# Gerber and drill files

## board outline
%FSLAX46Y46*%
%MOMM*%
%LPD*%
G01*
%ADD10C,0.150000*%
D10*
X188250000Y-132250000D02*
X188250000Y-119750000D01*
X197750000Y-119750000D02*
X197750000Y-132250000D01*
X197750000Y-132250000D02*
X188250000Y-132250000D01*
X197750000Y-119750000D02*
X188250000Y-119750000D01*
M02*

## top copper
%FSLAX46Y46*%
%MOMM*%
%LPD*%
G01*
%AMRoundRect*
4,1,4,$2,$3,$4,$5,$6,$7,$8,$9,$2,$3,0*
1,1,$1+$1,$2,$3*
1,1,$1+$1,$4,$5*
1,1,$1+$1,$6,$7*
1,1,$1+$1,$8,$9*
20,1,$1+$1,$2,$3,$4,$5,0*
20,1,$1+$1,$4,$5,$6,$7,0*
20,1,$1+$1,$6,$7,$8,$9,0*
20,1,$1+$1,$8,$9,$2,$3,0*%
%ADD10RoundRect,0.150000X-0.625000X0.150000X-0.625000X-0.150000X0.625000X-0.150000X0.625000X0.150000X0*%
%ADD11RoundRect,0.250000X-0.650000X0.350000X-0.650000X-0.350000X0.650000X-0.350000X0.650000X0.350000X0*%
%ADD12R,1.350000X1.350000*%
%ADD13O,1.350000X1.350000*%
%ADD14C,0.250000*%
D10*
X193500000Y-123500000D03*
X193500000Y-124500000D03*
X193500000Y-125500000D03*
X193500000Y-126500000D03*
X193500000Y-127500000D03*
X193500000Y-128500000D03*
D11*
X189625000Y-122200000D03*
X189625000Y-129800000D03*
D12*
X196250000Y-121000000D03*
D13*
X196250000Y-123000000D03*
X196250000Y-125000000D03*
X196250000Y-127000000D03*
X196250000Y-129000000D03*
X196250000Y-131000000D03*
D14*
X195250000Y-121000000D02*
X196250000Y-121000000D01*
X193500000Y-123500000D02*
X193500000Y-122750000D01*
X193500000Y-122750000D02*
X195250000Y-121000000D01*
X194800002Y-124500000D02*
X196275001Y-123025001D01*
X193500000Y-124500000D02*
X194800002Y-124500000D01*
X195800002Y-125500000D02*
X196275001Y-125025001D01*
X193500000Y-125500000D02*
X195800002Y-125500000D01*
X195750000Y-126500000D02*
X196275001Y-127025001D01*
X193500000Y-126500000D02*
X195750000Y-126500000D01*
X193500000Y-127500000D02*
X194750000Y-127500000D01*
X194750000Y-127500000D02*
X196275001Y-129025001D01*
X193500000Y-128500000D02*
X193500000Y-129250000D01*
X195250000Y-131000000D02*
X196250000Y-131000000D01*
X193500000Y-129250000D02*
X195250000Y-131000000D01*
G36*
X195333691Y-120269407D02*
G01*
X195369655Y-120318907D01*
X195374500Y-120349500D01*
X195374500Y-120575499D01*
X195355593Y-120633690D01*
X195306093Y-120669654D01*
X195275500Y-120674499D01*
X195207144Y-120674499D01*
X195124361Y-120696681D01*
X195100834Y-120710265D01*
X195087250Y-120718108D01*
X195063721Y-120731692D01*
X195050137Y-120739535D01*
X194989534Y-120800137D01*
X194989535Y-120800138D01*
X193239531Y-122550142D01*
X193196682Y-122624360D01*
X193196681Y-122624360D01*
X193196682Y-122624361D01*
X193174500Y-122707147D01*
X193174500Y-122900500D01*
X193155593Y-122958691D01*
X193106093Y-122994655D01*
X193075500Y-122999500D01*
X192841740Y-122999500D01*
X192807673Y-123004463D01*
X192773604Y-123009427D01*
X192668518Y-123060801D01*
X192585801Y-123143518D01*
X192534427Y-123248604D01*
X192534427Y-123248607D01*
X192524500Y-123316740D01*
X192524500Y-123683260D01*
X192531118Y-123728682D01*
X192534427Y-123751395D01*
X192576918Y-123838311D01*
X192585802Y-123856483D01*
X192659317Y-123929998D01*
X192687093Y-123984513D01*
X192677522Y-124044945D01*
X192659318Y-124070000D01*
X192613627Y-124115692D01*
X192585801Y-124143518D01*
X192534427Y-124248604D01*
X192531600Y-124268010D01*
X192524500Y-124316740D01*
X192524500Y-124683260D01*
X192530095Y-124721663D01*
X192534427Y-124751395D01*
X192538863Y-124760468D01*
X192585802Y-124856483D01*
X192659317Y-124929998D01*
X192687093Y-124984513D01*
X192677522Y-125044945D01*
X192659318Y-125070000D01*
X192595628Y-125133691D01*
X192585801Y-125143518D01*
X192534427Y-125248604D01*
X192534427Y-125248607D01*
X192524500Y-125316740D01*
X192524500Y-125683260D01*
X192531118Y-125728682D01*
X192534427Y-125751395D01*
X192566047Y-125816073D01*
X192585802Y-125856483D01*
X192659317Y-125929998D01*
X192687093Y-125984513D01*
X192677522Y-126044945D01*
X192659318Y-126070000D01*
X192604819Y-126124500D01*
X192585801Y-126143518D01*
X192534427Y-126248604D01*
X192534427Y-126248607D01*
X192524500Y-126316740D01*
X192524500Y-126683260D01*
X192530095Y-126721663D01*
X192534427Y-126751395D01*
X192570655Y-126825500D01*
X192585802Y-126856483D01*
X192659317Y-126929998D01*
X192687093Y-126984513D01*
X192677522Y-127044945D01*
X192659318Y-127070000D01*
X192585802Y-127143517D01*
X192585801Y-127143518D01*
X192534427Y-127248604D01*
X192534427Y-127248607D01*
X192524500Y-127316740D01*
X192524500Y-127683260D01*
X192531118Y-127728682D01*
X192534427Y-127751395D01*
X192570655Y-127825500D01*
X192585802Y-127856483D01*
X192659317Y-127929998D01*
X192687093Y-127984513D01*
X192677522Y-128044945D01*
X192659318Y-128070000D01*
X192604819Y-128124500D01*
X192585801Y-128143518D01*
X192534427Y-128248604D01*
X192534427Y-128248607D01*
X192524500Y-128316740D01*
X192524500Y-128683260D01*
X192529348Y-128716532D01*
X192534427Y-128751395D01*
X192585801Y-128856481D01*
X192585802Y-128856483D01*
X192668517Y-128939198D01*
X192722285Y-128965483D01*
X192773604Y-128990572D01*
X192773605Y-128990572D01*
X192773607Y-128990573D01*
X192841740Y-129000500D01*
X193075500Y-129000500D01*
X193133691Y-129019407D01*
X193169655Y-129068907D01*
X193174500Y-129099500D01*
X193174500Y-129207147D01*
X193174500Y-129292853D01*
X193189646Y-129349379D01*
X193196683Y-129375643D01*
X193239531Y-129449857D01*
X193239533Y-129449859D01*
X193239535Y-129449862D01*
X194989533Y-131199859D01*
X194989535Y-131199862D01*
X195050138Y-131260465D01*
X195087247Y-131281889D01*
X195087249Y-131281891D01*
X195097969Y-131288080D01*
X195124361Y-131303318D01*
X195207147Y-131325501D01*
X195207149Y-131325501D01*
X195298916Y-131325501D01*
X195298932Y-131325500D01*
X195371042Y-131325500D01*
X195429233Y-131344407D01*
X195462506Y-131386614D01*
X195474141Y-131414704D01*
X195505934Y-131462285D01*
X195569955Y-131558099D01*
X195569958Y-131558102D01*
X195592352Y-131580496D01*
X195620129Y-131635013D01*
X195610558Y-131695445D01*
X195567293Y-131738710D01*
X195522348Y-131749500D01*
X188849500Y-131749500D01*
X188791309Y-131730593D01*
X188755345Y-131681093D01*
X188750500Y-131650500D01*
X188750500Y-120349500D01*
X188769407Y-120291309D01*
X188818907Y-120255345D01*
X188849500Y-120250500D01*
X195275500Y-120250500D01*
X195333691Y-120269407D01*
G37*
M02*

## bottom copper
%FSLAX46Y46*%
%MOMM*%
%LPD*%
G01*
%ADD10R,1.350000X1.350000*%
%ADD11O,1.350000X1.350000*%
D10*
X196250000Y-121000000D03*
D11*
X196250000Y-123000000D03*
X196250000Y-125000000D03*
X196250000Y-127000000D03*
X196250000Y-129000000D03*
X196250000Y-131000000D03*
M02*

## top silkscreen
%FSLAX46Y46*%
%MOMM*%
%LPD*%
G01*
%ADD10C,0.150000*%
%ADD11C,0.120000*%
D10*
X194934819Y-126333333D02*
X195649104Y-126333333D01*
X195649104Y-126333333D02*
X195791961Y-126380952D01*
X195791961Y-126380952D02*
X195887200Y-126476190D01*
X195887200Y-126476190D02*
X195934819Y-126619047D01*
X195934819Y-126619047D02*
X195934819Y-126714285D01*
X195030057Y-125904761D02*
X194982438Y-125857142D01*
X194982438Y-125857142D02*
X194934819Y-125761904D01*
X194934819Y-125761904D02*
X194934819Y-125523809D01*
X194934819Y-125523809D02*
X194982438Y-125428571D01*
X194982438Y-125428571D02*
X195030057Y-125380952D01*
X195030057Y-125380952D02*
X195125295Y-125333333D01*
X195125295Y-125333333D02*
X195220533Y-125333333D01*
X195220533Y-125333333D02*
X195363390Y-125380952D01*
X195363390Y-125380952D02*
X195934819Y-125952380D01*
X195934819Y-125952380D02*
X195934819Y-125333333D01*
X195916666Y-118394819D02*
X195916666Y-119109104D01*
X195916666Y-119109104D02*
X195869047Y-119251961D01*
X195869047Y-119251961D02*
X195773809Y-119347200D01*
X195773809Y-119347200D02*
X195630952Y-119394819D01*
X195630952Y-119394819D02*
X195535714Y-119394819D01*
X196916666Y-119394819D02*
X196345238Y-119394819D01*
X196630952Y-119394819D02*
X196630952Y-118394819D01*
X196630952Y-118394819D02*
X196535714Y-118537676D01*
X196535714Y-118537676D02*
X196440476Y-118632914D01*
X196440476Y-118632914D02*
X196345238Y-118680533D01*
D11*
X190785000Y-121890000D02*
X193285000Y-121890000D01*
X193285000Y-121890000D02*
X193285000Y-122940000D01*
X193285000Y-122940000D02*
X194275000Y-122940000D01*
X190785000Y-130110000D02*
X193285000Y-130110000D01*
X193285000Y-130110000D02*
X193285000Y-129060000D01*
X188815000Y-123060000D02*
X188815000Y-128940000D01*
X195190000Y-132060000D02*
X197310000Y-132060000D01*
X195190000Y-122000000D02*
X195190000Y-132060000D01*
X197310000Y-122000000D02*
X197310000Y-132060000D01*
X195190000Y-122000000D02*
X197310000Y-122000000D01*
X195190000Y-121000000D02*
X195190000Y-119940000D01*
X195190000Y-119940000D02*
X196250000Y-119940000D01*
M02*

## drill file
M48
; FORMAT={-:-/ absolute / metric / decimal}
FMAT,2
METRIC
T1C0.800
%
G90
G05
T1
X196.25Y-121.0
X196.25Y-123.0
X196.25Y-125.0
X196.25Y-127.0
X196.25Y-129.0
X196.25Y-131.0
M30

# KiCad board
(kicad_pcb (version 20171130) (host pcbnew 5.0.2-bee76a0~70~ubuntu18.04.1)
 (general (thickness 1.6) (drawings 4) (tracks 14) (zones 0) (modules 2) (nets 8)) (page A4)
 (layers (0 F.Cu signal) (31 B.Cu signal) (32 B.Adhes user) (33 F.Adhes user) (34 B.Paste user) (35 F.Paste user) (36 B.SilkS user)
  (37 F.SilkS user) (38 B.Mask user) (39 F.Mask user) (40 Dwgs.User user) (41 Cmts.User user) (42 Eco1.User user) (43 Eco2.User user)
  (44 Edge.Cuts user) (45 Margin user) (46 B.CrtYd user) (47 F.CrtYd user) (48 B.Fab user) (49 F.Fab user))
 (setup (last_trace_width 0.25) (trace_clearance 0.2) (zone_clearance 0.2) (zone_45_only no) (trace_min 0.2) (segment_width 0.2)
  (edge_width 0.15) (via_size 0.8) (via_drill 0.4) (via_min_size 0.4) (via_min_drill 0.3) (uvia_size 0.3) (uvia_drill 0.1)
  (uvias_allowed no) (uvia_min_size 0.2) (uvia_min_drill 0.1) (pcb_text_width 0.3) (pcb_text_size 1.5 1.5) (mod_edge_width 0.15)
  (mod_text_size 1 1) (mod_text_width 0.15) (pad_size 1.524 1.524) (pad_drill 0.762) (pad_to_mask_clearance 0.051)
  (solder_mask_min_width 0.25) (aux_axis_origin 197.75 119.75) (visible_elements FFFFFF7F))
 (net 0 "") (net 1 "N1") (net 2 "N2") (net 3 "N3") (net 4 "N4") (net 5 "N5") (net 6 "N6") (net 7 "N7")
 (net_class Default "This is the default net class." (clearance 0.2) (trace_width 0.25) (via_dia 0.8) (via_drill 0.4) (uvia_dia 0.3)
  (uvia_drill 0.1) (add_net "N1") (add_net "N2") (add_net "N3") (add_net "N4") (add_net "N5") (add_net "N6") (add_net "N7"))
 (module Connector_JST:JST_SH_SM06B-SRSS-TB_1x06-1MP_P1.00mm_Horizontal (layer F.Cu) (at 191.5 126 270)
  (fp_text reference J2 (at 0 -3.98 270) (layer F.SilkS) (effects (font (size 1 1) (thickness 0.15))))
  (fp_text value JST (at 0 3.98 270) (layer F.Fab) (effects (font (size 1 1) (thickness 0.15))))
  (fp_line (start -4.11 0.715) (end -4.11 -1.785) (layer F.SilkS) (width 0.12))
  (fp_line (start -4.11 -1.785) (end -3.06 -1.785) (layer F.SilkS) (width 0.12))
  (fp_line (start -3.06 -1.785) (end -3.06 -2.775) (layer F.SilkS) (width 0.12))
  (fp_line (start 4.11 0.715) (end 4.11 -1.785) (layer F.SilkS) (width 0.12))
  (fp_line (start 4.11 -1.785) (end 3.06 -1.785) (layer F.SilkS) (width 0.12))
  (fp_line (start -2.94 2.685) (end 2.94 2.685) (layer F.SilkS) (width 0.12))
  (pad 1 smd roundrect (at -2.5 -2 270) (size 0.6 1.55) (layers F.Cu F.Paste F.Mask) (roundrect_rratio 0.25) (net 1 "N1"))
  (pad 2 smd roundrect (at -1.5 -2 270) (size 0.6 1.55) (layers F.Cu F.Paste F.Mask) (roundrect_rratio 0.25) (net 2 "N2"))
  (pad 3 smd roundrect (at -0.5 -2 270) (size 0.6 1.55) (layers F.Cu F.Paste F.Mask) (roundrect_rratio 0.25) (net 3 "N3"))
  (pad 4 smd roundrect (at 0.5 -2 270) (size 0.6 1.55) (layers F.Cu F.Paste F.Mask) (roundrect_rratio 0.25) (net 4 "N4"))
  (pad 5 smd roundrect (at 1.5 -2 270) (size 0.6 1.55) (layers F.Cu F.Paste F.Mask) (roundrect_rratio 0.25) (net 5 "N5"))
  (pad 6 smd roundrect (at 2.5 -2 270) (size 0.6 1.55) (layers F.Cu F.Paste F.Mask) (roundrect_rratio 0.25) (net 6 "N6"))
  (pad MP smd roundrect (at -3.8 1.875 270) (size 1.2 1.8) (layers F.Cu F.Paste F.Mask) (roundrect_rratio 0.208333) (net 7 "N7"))
  (pad MP smd roundrect (at 3.8 1.875 270) (size 1.2 1.8) (layers F.Cu F.Paste F.Mask) (roundrect_rratio 0.208333) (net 7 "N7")))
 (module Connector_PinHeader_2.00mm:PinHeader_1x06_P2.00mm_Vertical (layer F.Cu) (at 196.25 121)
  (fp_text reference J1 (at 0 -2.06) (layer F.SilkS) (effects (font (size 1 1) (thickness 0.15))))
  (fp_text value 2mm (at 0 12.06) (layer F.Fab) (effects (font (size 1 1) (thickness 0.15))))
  (fp_line (start -1.06 11.06) (end 1.06 11.06) (layer F.SilkS) (width 0.12))
  (fp_line (start -1.06 1) (end -1.06 11.06) (layer F.SilkS) (width 0.12))
  (fp_line (start 1.06 1) (end 1.06 11.06) (layer F.SilkS) (width 0.12))
  (fp_line (start -1.06 1) (end 1.06 1) (layer F.SilkS) (width 0.12))
  (fp_line (start -1.06 0) (end -1.06 -1.06) (layer F.SilkS) (width 0.12))
  (fp_line (start -1.06 -1.06) (end 0 -1.06) (layer F.SilkS) (width 0.12))
  (pad 1 thru_hole rect (at 0 0) (size 1.35 1.35) (drill 0.8) (layers *.Cu *.Mask) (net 1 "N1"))
  (pad 2 thru_hole oval (at 0 2) (size 1.35 1.35) (drill 0.8) (layers *.Cu *.Mask) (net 2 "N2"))
  (pad 3 thru_hole oval (at 0 4) (size 1.35 1.35) (drill 0.8) (layers *.Cu *.Mask) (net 3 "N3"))
  (pad 4 thru_hole oval (at 0 6) (size 1.35 1.35) (drill 0.8) (layers *.Cu *.Mask) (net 4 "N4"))
  (pad 5 thru_hole oval (at 0 8) (size 1.35 1.35) (drill 0.8) (layers *.Cu *.Mask) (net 5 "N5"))
  (pad 6 thru_hole oval (at 0 10) (size 1.35 1.35) (drill 0.8) (layers *.Cu *.Mask) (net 6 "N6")))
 (gr_line (start 188.25 132.25) (end 188.25 119.75) (layer Edge.Cuts) (width 0.15))
 (gr_line (start 197.75 119.75) (end 197.75 132.25) (layer Edge.Cuts) (width 0.15))
 (gr_line (start 197.75 132.25) (end 188.25 132.25) (layer Edge.Cuts) (width 0.15))
 (gr_line (start 197.75 119.75) (end 188.25 119.75) (layer Edge.Cuts) (width 0.15))
 (segment (start 195.25 121) (end 196.25 121) (width 0.25) (layer F.Cu) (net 1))
 (segment (start 193.5 123.5) (end 193.5 122.75) (width 0.25) (layer F.Cu) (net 1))
 (segment (start 193.5 122.75) (end 195.25 121) (width 0.25) (layer F.Cu) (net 1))
 (segment (start 194.800002 124.5) (end 196.275001 123.025001) (width 0.25) (layer F.Cu) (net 2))
 (segment (start 193.5 124.5) (end 194.800002 124.5) (width 0.25) (layer F.Cu) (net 2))
 (segment (start 195.800002 125.5) (end 196.275001 125.025001) (width 0.25) (layer F.Cu) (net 3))
 (segment (start 193.5 125.5) (end 195.800002 125.5) (width 0.25) (layer F.Cu) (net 3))
 (segment (start 195.75 126.5) (end 196.275001 127.025001) (width 0.25) (layer F.Cu) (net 4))
 (segment (start 193.5 126.5) (end 195.75 126.5) (width 0.25) (layer F.Cu) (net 4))
 (segment (start 193.5 127.5) (end 194.75 127.5) (width 0.25) (layer F.Cu) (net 5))
 (segment (start 194.75 127.5) (end 196.275001 129.025001) (width 0.25) (layer F.Cu) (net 5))
 (segment (start 193.5 128.5) (end 193.5 129.25) (width 0.25) (layer F.Cu) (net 6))
 (segment (start 195.25 131) (end 196.25 131) (width 0.25) (layer F.Cu) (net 6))
 (segment (start 193.5 129.25) (end 195.25 131) (width 0.25) (layer F.Cu) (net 6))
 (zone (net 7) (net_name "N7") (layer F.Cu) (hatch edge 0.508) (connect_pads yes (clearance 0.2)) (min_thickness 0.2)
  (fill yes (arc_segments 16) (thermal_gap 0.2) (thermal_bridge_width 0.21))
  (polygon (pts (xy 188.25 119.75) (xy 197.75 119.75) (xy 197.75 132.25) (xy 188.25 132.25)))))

